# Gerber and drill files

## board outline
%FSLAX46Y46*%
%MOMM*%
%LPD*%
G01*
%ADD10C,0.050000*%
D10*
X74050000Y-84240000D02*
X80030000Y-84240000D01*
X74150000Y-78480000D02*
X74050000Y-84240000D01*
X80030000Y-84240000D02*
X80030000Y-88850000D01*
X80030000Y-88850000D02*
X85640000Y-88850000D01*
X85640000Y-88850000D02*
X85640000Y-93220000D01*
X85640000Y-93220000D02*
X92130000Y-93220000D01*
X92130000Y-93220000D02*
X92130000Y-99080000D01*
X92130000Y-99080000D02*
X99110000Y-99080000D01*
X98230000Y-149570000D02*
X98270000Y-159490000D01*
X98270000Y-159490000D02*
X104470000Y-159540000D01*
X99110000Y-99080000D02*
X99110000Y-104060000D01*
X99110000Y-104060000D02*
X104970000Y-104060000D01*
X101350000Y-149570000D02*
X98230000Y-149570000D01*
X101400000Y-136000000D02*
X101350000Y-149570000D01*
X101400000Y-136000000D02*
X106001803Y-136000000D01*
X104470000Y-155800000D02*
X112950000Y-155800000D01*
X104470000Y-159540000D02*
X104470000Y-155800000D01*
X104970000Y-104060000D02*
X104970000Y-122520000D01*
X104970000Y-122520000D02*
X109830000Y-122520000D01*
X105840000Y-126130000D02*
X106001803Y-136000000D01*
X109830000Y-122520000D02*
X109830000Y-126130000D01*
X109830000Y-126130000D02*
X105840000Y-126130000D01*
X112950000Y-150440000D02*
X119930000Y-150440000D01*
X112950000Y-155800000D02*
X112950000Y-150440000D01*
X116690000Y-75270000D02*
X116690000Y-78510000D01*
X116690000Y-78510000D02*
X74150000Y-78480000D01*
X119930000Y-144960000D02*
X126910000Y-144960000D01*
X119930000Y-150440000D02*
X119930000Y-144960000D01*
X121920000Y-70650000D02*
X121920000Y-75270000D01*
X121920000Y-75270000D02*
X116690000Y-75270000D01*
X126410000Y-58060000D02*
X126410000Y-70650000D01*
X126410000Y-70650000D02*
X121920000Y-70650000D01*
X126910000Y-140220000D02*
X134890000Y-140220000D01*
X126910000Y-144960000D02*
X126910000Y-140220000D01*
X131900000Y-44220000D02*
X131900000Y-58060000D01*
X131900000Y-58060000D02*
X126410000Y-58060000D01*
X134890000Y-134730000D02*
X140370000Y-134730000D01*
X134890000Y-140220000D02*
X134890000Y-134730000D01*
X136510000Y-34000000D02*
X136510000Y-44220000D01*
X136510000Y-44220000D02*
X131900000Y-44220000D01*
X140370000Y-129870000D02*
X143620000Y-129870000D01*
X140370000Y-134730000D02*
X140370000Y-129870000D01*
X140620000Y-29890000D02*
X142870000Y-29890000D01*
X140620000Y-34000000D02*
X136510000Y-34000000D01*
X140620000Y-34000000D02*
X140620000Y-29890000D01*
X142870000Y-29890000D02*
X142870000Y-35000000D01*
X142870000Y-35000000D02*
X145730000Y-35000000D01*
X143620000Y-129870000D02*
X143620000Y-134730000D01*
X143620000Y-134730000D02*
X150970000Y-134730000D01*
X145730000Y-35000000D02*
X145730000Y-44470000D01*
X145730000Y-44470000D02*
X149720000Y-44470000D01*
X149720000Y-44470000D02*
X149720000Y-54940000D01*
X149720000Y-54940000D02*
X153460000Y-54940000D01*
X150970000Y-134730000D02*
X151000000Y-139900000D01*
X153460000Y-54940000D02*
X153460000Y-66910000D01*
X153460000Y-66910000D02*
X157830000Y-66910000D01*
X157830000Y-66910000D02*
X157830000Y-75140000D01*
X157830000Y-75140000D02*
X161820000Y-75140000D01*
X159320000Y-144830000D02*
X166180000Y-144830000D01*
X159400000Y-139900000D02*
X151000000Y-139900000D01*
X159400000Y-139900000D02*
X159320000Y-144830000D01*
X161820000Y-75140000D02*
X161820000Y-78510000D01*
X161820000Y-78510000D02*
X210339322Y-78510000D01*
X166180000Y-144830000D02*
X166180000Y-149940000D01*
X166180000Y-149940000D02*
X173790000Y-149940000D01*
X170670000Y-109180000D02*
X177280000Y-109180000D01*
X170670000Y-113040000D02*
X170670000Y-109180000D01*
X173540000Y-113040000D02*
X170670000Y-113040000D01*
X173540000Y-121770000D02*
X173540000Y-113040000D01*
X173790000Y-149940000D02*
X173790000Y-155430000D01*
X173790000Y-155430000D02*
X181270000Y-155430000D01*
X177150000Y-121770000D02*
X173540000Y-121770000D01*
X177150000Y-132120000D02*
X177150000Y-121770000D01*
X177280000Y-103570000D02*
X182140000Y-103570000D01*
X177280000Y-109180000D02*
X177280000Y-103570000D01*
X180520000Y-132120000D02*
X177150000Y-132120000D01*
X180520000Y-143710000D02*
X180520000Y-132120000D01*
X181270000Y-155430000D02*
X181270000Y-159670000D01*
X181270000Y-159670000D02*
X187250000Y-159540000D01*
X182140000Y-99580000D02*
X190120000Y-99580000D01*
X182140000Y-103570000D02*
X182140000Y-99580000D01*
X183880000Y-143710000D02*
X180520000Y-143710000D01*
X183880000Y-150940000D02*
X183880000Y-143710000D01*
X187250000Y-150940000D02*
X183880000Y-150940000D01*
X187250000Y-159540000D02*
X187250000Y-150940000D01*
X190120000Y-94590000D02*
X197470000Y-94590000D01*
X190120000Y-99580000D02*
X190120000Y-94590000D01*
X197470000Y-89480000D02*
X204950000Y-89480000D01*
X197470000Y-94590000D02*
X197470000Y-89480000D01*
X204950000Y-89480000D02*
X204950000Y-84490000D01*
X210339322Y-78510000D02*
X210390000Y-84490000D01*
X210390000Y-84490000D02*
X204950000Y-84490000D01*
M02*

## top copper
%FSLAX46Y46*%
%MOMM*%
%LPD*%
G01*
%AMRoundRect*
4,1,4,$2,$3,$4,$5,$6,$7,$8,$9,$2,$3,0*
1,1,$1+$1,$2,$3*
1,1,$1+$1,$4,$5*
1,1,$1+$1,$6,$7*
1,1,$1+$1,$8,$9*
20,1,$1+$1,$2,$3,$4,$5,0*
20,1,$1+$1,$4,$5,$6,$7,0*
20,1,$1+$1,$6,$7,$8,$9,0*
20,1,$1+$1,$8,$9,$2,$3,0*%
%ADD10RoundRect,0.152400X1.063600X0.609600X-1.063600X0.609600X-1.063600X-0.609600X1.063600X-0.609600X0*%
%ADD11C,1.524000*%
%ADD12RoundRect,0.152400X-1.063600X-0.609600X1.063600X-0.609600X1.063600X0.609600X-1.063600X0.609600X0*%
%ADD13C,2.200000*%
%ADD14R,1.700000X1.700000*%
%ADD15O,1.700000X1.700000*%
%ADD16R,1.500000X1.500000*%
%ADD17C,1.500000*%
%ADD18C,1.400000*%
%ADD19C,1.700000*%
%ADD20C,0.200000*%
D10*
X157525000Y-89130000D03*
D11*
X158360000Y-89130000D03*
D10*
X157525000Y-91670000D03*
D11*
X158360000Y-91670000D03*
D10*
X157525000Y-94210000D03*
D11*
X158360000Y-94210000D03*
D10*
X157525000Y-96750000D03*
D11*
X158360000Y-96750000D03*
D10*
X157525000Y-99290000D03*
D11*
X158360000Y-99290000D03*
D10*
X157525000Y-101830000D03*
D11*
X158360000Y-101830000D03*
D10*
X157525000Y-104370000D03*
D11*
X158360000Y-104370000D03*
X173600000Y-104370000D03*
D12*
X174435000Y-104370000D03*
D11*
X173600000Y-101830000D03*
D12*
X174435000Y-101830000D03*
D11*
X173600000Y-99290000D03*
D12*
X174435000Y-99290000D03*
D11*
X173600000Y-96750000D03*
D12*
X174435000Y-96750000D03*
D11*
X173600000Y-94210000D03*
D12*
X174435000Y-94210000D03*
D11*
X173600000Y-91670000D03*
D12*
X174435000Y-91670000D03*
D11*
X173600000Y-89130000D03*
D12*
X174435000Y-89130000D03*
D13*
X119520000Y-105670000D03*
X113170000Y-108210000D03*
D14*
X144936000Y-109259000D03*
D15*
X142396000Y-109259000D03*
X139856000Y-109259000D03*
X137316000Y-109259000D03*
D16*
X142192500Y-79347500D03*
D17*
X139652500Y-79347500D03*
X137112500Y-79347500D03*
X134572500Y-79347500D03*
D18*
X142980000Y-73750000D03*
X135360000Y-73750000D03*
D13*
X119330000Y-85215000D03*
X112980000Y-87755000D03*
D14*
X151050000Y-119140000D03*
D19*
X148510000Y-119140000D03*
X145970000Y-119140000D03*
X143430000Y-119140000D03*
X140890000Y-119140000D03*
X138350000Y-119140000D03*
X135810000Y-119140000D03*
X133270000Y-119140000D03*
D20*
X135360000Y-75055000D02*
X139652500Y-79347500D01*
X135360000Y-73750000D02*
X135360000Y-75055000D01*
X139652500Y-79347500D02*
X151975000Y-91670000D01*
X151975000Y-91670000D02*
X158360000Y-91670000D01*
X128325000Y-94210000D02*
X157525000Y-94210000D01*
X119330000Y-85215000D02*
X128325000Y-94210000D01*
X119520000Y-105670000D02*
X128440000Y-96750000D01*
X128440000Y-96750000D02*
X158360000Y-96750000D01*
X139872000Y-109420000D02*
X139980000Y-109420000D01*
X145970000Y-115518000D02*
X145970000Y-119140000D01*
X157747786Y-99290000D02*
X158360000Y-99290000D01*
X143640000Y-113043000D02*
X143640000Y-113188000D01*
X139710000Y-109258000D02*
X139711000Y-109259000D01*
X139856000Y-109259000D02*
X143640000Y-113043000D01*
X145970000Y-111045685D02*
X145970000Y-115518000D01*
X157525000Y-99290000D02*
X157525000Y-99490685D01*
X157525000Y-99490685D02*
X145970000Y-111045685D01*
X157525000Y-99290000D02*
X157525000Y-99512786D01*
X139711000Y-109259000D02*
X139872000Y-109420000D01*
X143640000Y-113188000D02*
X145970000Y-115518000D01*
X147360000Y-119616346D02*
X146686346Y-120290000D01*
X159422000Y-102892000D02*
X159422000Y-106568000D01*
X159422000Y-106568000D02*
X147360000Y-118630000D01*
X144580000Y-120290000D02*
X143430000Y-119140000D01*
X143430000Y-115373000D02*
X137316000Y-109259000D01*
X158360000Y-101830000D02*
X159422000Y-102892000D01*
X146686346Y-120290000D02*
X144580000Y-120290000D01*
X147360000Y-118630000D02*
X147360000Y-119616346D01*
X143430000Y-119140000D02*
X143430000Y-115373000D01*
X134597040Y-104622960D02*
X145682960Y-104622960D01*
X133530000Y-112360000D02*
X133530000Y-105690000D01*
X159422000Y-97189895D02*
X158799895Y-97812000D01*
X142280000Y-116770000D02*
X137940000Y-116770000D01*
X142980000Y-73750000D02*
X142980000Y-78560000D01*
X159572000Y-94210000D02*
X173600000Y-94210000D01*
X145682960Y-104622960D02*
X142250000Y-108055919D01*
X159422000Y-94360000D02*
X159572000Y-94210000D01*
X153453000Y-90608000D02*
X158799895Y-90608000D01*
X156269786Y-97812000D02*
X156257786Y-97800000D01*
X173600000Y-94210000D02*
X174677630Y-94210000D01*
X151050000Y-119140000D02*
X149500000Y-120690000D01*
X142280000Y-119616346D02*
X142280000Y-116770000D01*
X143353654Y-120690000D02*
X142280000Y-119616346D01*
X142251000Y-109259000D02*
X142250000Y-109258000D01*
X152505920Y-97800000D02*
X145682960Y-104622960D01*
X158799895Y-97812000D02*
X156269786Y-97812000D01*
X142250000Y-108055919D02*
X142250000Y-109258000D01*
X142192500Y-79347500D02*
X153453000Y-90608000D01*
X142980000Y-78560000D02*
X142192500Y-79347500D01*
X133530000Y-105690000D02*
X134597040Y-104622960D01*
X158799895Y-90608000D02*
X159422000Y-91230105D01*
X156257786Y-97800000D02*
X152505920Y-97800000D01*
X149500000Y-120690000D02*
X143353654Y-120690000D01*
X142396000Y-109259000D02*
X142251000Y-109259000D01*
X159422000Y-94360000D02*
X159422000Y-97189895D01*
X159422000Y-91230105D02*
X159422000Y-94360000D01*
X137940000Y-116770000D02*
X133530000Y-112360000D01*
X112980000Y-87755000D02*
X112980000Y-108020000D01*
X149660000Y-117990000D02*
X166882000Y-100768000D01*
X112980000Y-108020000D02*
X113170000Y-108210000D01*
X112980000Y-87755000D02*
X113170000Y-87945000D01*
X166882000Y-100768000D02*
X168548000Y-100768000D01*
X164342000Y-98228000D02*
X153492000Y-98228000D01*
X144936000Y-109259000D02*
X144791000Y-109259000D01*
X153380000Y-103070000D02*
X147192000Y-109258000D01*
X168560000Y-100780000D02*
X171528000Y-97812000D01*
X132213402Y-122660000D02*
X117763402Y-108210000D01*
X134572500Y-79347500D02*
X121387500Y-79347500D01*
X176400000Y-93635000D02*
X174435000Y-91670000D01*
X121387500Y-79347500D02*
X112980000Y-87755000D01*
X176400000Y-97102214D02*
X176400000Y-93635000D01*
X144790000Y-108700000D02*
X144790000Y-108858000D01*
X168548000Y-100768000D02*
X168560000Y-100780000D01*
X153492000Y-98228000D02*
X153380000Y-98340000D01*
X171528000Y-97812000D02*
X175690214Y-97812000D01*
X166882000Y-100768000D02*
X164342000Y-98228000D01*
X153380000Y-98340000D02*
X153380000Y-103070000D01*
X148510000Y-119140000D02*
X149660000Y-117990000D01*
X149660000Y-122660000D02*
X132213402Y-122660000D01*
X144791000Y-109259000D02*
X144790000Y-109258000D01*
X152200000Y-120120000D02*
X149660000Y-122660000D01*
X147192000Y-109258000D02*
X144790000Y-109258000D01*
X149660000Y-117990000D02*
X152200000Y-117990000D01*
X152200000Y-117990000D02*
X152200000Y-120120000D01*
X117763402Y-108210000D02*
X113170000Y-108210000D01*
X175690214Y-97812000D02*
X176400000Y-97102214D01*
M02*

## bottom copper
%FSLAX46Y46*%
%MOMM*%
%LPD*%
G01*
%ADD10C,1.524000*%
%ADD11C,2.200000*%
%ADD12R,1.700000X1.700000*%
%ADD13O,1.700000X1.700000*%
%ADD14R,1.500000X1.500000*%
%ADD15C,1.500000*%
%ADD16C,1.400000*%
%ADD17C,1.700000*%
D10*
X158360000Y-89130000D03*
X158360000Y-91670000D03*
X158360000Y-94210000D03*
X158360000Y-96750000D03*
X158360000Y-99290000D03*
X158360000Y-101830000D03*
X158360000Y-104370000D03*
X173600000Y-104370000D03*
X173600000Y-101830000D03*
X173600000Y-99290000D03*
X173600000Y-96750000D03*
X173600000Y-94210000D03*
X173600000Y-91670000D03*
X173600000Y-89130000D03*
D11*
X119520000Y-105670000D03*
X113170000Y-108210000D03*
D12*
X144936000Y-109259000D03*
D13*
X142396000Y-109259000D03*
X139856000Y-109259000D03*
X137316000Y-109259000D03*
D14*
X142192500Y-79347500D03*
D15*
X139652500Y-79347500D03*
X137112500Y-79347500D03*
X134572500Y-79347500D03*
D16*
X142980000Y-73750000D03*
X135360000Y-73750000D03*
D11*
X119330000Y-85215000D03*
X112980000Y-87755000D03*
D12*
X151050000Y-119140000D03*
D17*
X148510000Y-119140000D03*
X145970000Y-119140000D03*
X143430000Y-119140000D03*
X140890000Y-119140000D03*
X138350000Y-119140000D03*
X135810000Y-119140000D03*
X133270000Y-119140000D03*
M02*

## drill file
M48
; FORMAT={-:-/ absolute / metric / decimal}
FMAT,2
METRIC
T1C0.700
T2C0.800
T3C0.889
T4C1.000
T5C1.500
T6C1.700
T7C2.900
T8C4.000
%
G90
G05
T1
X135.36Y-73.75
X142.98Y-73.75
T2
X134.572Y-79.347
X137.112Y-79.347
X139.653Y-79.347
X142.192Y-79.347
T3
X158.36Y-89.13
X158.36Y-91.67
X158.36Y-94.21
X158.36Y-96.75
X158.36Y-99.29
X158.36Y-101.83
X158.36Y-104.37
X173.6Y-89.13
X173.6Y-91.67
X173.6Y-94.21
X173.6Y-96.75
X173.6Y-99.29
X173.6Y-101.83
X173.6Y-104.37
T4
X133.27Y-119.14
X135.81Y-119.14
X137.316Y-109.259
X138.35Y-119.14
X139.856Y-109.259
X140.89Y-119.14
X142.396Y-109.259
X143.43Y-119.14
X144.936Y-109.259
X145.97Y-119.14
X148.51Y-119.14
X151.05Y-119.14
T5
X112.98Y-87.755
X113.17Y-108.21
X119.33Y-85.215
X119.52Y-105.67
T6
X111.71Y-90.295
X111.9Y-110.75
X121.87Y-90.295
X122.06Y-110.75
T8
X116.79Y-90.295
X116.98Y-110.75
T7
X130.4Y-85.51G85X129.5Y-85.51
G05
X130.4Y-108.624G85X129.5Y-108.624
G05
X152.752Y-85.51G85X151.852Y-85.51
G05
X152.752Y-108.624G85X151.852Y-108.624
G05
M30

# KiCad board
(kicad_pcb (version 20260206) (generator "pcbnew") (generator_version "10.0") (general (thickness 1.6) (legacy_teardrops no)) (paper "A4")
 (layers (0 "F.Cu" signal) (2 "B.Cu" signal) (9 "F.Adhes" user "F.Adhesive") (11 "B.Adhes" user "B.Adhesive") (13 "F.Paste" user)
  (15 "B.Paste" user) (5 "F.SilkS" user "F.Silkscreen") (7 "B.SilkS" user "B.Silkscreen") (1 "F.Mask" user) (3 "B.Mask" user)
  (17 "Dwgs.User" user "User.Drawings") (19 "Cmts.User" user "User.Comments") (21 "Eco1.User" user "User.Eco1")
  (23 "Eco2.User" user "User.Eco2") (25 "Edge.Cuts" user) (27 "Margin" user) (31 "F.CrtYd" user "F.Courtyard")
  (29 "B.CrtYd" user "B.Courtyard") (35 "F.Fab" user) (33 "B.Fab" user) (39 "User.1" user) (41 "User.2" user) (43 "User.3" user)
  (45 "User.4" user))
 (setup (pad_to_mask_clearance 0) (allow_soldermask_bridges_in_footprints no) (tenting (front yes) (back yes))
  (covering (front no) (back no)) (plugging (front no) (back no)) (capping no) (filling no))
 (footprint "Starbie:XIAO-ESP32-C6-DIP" (layer "F.Cu") (at 165.98 96.75 90)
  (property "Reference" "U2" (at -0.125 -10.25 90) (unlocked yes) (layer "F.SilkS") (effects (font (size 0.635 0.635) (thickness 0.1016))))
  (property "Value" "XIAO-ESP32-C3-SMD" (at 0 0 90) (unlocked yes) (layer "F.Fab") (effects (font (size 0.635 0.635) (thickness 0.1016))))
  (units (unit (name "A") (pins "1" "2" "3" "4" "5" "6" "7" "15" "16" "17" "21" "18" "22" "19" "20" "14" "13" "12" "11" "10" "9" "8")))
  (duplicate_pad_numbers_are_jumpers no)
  (pad "1" smd roundrect (at 7.62 -8.455 180) (size 2.432 1.524) (layers "F.Cu" "F.Mask") (roundrect_rratio 0.1)
   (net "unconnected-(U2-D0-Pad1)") (thermal_bridge_angle 45))
  (pad "1" thru_hole circle (at 7.62 -7.62 180) (size 1.524 1.524) (drill 0.889) (layers "*.Cu" "*.Mask") (remove_unused_layers no)
   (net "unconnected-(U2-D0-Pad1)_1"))
  (pad "2" smd roundrect (at 5.08 -8.455 180) (size 2.432 1.524) (layers "F.Cu" "F.Mask") (roundrect_rratio 0.1) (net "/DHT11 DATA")
   (thermal_bridge_angle 45))
  (pad "2" thru_hole circle (at 5.08 -7.62 180) (size 1.524 1.524) (drill 0.889) (layers "*.Cu" "*.Mask") (remove_unused_layers no)
   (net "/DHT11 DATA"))
  (pad "3" smd roundrect (at 2.54 -8.455 180) (size 2.432 1.524) (layers "F.Cu" "F.Mask") (roundrect_rratio 0.1) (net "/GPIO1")
   (thermal_bridge_angle 45))
  (pad "3" thru_hole circle (at 2.54 -7.62 180) (size 1.524 1.524) (drill 0.889) (layers "*.Cu" "*.Mask") (remove_unused_layers no)
   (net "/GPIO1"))
  (pad "4" smd roundrect (at 0 -8.455 180) (size 2.432 1.524) (layers "F.Cu" "F.Mask") (roundrect_rratio 0.1) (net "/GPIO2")
   (thermal_bridge_angle 45))
  (pad "4" thru_hole circle (at 0 -7.62 180) (size 1.524 1.524) (drill 0.889) (layers "*.Cu" "*.Mask") (remove_unused_layers no)
   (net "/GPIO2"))
  (pad "5" smd roundrect (at -2.54 -8.455 180) (size 2.432 1.524) (layers "F.Cu" "F.Mask") (roundrect_rratio 0.1) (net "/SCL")
   (thermal_bridge_angle 45))
  (pad "5" thru_hole circle (at -2.54 -7.62 180) (size 1.524 1.524) (drill 0.889) (layers "*.Cu" "*.Mask") (remove_unused_layers no)
   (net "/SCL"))
  (pad "6" smd roundrect (at -5.08 -8.455 180) (size 2.432 1.524) (layers "F.Cu" "F.Mask") (roundrect_rratio 0.1) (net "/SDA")
   (thermal_bridge_angle 45))
  (pad "6" thru_hole circle (at -5.08 -7.62 180) (size 1.524 1.524) (drill 0.889) (layers "*.Cu" "*.Mask") (remove_unused_layers no)
   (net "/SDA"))
  (pad "7" smd roundrect (at -7.62 -8.455 180) (size 2.432 1.524) (layers "F.Cu" "F.Mask") (roundrect_rratio 0.1)
   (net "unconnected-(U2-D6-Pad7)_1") (thermal_bridge_angle 45))
  (pad "7" thru_hole circle (at -7.62 -7.62 180) (size 1.524 1.524) (drill 0.889) (layers "*.Cu" "*.Mask") (remove_unused_layers no)
   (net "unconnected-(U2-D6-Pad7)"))
  (pad "8" thru_hole circle (at -7.62 7.62) (size 1.524 1.524) (drill 0.889) (layers "*.Cu" "*.Mask") (remove_unused_layers no)
   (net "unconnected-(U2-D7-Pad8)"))
  (pad "8" smd roundrect (at -7.62 8.455) (size 2.432 1.524) (layers "F.Cu" "F.Mask") (roundrect_rratio 0.1)
   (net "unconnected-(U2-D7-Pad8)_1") (thermal_bridge_angle 45))
  (pad "9" thru_hole circle (at -5.08 7.62) (size 1.524 1.524) (drill 0.889) (layers "*.Cu" "*.Mask") (remove_unused_layers no)
   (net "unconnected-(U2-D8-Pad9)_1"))
  (pad "9" smd roundrect (at -5.08 8.455) (size 2.432 1.524) (layers "F.Cu" "F.Mask") (roundrect_rratio 0.1)
   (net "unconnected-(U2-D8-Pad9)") (thermal_bridge_angle 45))
  (pad "10" thru_hole circle (at -2.54 7.62) (size 1.524 1.524) (drill 0.889) (layers "*.Cu" "*.Mask") (remove_unused_layers no)
   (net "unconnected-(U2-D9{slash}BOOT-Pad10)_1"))
  (pad "10" smd roundrect (at -2.54 8.455) (size 2.432 1.524) (layers "F.Cu" "F.Mask") (roundrect_rratio 0.1)
   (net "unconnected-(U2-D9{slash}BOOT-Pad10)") (thermal_bridge_angle 45))
  (pad "11" thru_hole circle (at 0 7.62) (size 1.524 1.524) (drill 0.889) (layers "*.Cu" "*.Mask") (remove_unused_layers no)
   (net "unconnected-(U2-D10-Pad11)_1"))
  (pad "11" smd roundrect (at 0 8.455) (size 2.432 1.524) (layers "F.Cu" "F.Mask") (roundrect_rratio 0.1) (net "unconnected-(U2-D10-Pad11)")
   (thermal_bridge_angle 45))
  (pad "12" thru_hole circle (at 2.54 7.62) (size 1.524 1.524) (drill 0.889) (layers "*.Cu" "*.Mask") (remove_unused_layers no)
   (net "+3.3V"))
  (pad "12" smd roundrect (at 2.54 8.455) (size 2.432 1.524) (layers "F.Cu" "F.Mask") (roundrect_rratio 0.1) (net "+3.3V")
   (thermal_bridge_angle 45))
  (pad "13" thru_hole circle (at 5.08 7.62) (size 1.524 1.524) (drill 0.889) (layers "*.Cu" "*.Mask") (remove_unused_layers no) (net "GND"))
  (pad "13" smd roundrect (at 5.08 8.455) (size 2.432 1.524) (layers "F.Cu" "F.Mask") (roundrect_rratio 0.1) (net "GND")
   (thermal_bridge_angle 45))
  (pad "14" thru_hole circle (at 7.62 7.62) (size 1.524 1.524) (drill 0.889) (layers "*.Cu" "*.Mask") (remove_unused_layers no) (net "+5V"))
  (pad "14" smd roundrect (at 7.62 8.455) (size 2.432 1.524) (layers "F.Cu" "F.Mask") (roundrect_rratio 0.1) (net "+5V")
   (thermal_bridge_angle 45)))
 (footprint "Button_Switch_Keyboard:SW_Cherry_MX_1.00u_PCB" (layer "F.Cu") (at 119.52 105.67)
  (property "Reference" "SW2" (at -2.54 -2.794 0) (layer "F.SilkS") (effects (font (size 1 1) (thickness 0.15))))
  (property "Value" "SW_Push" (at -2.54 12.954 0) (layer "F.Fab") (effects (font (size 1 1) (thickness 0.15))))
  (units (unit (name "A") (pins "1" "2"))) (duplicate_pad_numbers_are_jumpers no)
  (pad "" np_thru_hole circle (at -7.62 5.08) (size 1.7 1.7) (drill 1.7) (layers "*.Cu" "*.Mask"))
  (pad "" np_thru_hole circle (at -2.54 5.08) (size 4 4) (drill 4) (layers "*.Cu" "*.Mask"))
  (pad "" np_thru_hole circle (at 2.54 5.08) (size 1.7 1.7) (drill 1.7) (layers "*.Cu" "*.Mask"))
  (pad "1" thru_hole circle (at 0 0) (size 2.2 2.2) (drill 1.5) (layers "*.Cu" "*.Mask") (remove_unused_layers no) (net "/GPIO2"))
  (pad "2" thru_hole circle (at -6.35 2.54) (size 2.2 2.2) (drill 1.5) (layers "*.Cu" "*.Mask") (remove_unused_layers no) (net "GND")))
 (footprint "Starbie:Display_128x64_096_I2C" (layer "F.Cu") (at 141.126 109.259 180)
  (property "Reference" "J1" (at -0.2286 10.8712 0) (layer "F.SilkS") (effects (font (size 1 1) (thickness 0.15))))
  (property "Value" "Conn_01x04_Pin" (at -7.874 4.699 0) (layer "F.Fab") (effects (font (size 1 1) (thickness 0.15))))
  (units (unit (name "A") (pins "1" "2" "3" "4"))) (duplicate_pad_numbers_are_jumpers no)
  (pad "" np_thru_hole oval (at -11.176 0.635 180) (size 3.8 2.9) (drill oval 3.8 2.9) (layers "*.Cu" "*.Mask"))
  (pad "" np_thru_hole oval (at -11.176 23.749 180) (size 3.8 2.9) (drill oval 3.8 2.9) (layers "*.Cu" "*.Mask"))
  (pad "" np_thru_hole oval (at 11.176 0.635 180) (size 3.8 2.9) (drill oval 3.8 2.9) (layers "*.Cu" "*.Mask"))
  (pad "" np_thru_hole oval (at 11.176 23.749 180) (size 3.8 2.9) (drill oval 3.8 2.9) (layers "*.Cu" "*.Mask"))
  (pad "1" thru_hole rect (at -3.81 0 270) (size 1.7 1.7) (drill 1) (layers "*.Cu" "*.Mask") (remove_unused_layers no) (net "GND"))
  (pad "2" thru_hole oval (at -1.27 0 270) (size 1.7 1.7) (drill 1) (layers "*.Cu" "*.Mask") (remove_unused_layers no) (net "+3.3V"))
  (pad "3" thru_hole oval (at 1.27 0 270) (size 1.7 1.7) (drill 1) (layers "*.Cu" "*.Mask") (remove_unused_layers no) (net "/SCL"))
  (pad "4" thru_hole oval (at 3.81 0 270) (size 1.7 1.7) (drill 1) (layers "*.Cu" "*.Mask") (remove_unused_layers no) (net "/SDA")))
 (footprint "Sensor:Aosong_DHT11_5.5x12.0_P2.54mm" (layer "F.Cu") (at 142.1925 79.3475 -90)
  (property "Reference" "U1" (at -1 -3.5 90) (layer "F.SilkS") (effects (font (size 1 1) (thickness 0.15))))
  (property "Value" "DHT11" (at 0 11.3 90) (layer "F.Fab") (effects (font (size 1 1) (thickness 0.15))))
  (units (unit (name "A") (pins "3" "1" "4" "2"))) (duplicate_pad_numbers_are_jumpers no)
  (pad "1" thru_hole rect (at 0 0 270) (size 1.5 1.5) (drill 0.8) (layers "*.Cu" "*.Mask") (remove_unused_layers no) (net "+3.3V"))
  (pad "2" thru_hole circle (at 0 2.54 270) (size 1.5 1.5) (drill 0.8) (layers "*.Cu" "*.Mask") (remove_unused_layers no)
   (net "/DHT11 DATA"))
  (pad "3" thru_hole circle (at 0 5.08 270) (size 1.5 1.5) (drill 0.8) (layers "*.Cu" "*.Mask") (remove_unused_layers no)
   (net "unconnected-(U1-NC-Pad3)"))
  (pad "4" thru_hole circle (at 0 7.62 270) (size 1.5 1.5) (drill 0.8) (layers "*.Cu" "*.Mask") (remove_unused_layers no) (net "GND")))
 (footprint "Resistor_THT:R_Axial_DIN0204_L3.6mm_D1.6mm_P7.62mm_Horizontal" (layer "F.Cu") (at 142.98 73.75 180)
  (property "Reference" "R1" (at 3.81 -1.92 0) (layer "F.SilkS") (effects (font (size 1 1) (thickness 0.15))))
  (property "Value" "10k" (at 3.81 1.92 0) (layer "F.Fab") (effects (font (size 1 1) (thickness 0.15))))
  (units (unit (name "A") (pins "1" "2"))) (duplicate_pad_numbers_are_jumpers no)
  (pad "1" thru_hole circle (at 0 0 180) (size 1.4 1.4) (drill 0.7) (layers "*.Cu" "*.Mask") (remove_unused_layers no) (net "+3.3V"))
  (pad "2" thru_hole circle (at 7.62 0 180) (size 1.4 1.4) (drill 0.7) (layers "*.Cu" "*.Mask") (remove_unused_layers no)
   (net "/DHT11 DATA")))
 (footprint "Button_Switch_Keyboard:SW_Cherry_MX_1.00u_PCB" (layer "F.Cu") (at 119.33 85.215)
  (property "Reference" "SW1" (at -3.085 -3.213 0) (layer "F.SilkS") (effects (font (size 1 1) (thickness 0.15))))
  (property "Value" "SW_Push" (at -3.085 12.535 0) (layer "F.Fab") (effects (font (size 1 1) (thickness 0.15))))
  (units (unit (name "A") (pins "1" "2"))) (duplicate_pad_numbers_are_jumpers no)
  (pad "" np_thru_hole circle (at -7.62 5.08) (size 1.7 1.7) (drill 1.7) (layers "*.Cu" "*.Mask"))
  (pad "" np_thru_hole circle (at -2.54 5.08) (size 4 4) (drill 4) (layers "*.Cu" "*.Mask"))
  (pad "" np_thru_hole circle (at 2.54 5.08) (size 1.7 1.7) (drill 1.7) (layers "*.Cu" "*.Mask"))
  (pad "1" thru_hole circle (at 0 0) (size 2.2 2.2) (drill 1.5) (layers "*.Cu" "*.Mask") (remove_unused_layers no) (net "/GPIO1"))
  (pad "2" thru_hole circle (at -6.35 2.54) (size 2.2 2.2) (drill 1.5) (layers "*.Cu" "*.Mask") (remove_unused_layers no) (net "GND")))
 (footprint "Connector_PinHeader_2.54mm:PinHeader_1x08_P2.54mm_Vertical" (layer "F.Cu") (at 151.05 119.14 -90)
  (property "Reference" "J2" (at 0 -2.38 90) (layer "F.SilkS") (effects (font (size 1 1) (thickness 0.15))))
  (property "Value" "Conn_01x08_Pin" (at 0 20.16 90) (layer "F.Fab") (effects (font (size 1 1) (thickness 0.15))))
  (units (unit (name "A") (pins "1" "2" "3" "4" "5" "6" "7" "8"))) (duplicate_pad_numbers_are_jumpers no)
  (pad "1" thru_hole rect (at 0 0 270) (size 1.7 1.7) (drill 1) (layers "*.Cu" "*.Mask") (remove_unused_layers no) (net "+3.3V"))
  (pad "2" thru_hole circle (at 0 2.54 270) (size 1.7 1.7) (drill 1) (layers "*.Cu" "*.Mask") (remove_unused_layers no) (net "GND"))
  (pad "3" thru_hole circle (at 0 5.08 270) (size 1.7 1.7) (drill 1) (layers "*.Cu" "*.Mask") (remove_unused_layers no) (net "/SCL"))
  (pad "4" thru_hole circle (at 0 7.62 270) (size 1.7 1.7) (drill 1) (layers "*.Cu" "*.Mask") (remove_unused_layers no) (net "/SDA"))
  (pad "5" thru_hole circle (at 0 10.16 270) (size 1.7 1.7) (drill 1) (layers "*.Cu" "*.Mask") (remove_unused_layers no)
   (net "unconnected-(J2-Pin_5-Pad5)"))
  (pad "6" thru_hole circle (at 0 12.7 270) (size 1.7 1.7) (drill 1) (layers "*.Cu" "*.Mask") (remove_unused_layers no)
   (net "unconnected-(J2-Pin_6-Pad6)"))
  (pad "7" thru_hole circle (at 0 15.24 270) (size 1.7 1.7) (drill 1) (layers "*.Cu" "*.Mask") (remove_unused_layers no)
   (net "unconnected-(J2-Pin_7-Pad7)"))
  (pad "8" thru_hole circle (at 0 17.78 270) (size 1.7 1.7) (drill 1) (layers "*.Cu" "*.Mask") (remove_unused_layers no)
   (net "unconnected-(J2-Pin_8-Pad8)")))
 (gr_line (start 74.05 84.24) (end 80.03 84.24) (stroke (width 0.05) (type default)) (layer "Edge.Cuts"))
 (gr_line (start 74.15 78.48) (end 74.05 84.24) (stroke (width 0.05) (type default)) (layer "Edge.Cuts"))
 (gr_line (start 80.03 84.24) (end 80.03 88.85) (stroke (width 0.05) (type default)) (layer "Edge.Cuts"))
 (gr_line (start 80.03 88.85) (end 85.64 88.85) (stroke (width 0.05) (type default)) (layer "Edge.Cuts"))
 (gr_line (start 85.64 88.85) (end 85.64 93.22) (stroke (width 0.05) (type default)) (layer "Edge.Cuts"))
 (gr_line (start 85.64 93.22) (end 92.13 93.22) (stroke (width 0.05) (type default)) (layer "Edge.Cuts"))
 (gr_line (start 92.13 93.22) (end 92.13 99.08) (stroke (width 0.05) (type default)) (layer "Edge.Cuts"))
 (gr_line (start 92.13 99.08) (end 99.11 99.08) (stroke (width 0.05) (type default)) (layer "Edge.Cuts"))
 (gr_line (start 98.23 149.57) (end 98.27 159.49) (stroke (width 0.05) (type default)) (layer "Edge.Cuts"))
 (gr_line (start 98.27 159.49) (end 104.47 159.54) (stroke (width 0.05) (type default)) (layer "Edge.Cuts"))
 (gr_line (start 99.11 99.08) (end 99.11 104.06) (stroke (width 0.05) (type default)) (layer "Edge.Cuts"))
 (gr_line (start 99.11 104.06) (end 104.97 104.06) (stroke (width 0.05) (type default)) (layer "Edge.Cuts"))
 (gr_line (start 101.35 149.57) (end 98.23 149.57) (stroke (width 0.05) (type default)) (layer "Edge.Cuts"))
 (gr_line (start 101.4 136) (end 101.35 149.57) (stroke (width 0.05) (type default)) (layer "Edge.Cuts"))
 (gr_line (start 101.4 136) (end 106.001803 136) (stroke (width 0.05) (type default)) (layer "Edge.Cuts"))
 (gr_line (start 104.47 155.8) (end 112.95 155.8) (stroke (width 0.05) (type default)) (layer "Edge.Cuts"))
 (gr_line (start 104.47 159.54) (end 104.47 155.8) (stroke (width 0.05) (type default)) (layer "Edge.Cuts"))
 (gr_line (start 104.97 104.06) (end 104.97 122.52) (stroke (width 0.05) (type default)) (layer "Edge.Cuts"))
 (gr_line (start 104.97 122.52) (end 109.83 122.52) (stroke (width 0.05) (type default)) (layer "Edge.Cuts"))
 (gr_line (start 105.84 126.13) (end 106.001803 136) (stroke (width 0.05) (type default)) (layer "Edge.Cuts"))
 (gr_line (start 109.83 122.52) (end 109.83 126.13) (stroke (width 0.05) (type default)) (layer "Edge.Cuts"))
 (gr_line (start 109.83 126.13) (end 105.84 126.13) (stroke (width 0.05) (type default)) (layer "Edge.Cuts"))
 (gr_line (start 112.95 150.44) (end 119.93 150.44) (stroke (width 0.05) (type default)) (layer "Edge.Cuts"))
 (gr_line (start 112.95 155.8) (end 112.95 150.44) (stroke (width 0.05) (type default)) (layer "Edge.Cuts"))
 (gr_line (start 116.69 75.27) (end 116.69 78.51) (stroke (width 0.05) (type default)) (layer "Edge.Cuts"))
 (gr_line (start 116.69 78.51) (end 74.15 78.48) (stroke (width 0.05) (type default)) (layer "Edge.Cuts"))
 (gr_line (start 119.93 144.96) (end 126.91 144.96) (stroke (width 0.05) (type default)) (layer "Edge.Cuts"))
 (gr_line (start 119.93 150.44) (end 119.93 144.96) (stroke (width 0.05) (type default)) (layer "Edge.Cuts"))
 (gr_line (start 121.92 70.65) (end 121.92 75.27) (stroke (width 0.05) (type default)) (layer "Edge.Cuts"))
 (gr_line (start 121.92 75.27) (end 116.69 75.27) (stroke (width 0.05) (type default)) (layer "Edge.Cuts"))
 (gr_line (start 126.41 58.06) (end 126.41 70.65) (stroke (width 0.05) (type default)) (layer "Edge.Cuts"))
 (gr_line (start 126.41 70.65) (end 121.92 70.65) (stroke (width 0.05) (type default)) (layer "Edge.Cuts"))
 (gr_line (start 126.91 140.22) (end 134.89 140.22) (stroke (width 0.05) (type default)) (layer "Edge.Cuts"))
 (gr_line (start 126.91 144.96) (end 126.91 140.22) (stroke (width 0.05) (type default)) (layer "Edge.Cuts"))
 (gr_line (start 131.9 44.22) (end 131.9 58.06) (stroke (width 0.05) (type default)) (layer "Edge.Cuts"))
 (gr_line (start 131.9 58.06) (end 126.41 58.06) (stroke (width 0.05) (type default)) (layer "Edge.Cuts"))
 (gr_line (start 134.89 134.73) (end 140.37 134.73) (stroke (width 0.05) (type default)) (layer "Edge.Cuts"))
 (gr_line (start 134.89 140.22) (end 134.89 134.73) (stroke (width 0.05) (type default)) (layer "Edge.Cuts"))
 (gr_line (start 136.51 34) (end 136.51 44.22) (stroke (width 0.05) (type default)) (layer "Edge.Cuts"))
 (gr_line (start 136.51 44.22) (end 131.9 44.22) (stroke (width 0.05) (type default)) (layer "Edge.Cuts"))
 (gr_line (start 140.37 129.87) (end 143.62 129.87) (stroke (width 0.05) (type default)) (layer "Edge.Cuts"))
 (gr_line (start 140.37 134.73) (end 140.37 129.87) (stroke (width 0.05) (type default)) (layer "Edge.Cuts"))
 (gr_line (start 140.62 29.89) (end 142.87 29.89) (stroke (width 0.05) (type default)) (layer "Edge.Cuts"))
 (gr_line (start 140.62 34) (end 136.51 34) (stroke (width 0.05) (type default)) (layer "Edge.Cuts"))
 (gr_line (start 140.62 34) (end 140.62 29.89) (stroke (width 0.05) (type default)) (layer "Edge.Cuts"))
 (gr_line (start 142.87 29.89) (end 142.87 35) (stroke (width 0.05) (type default)) (layer "Edge.Cuts"))
 (gr_line (start 142.87 35) (end 145.73 35) (stroke (width 0.05) (type default)) (layer "Edge.Cuts"))
 (gr_line (start 143.62 129.87) (end 143.62 134.73) (stroke (width 0.05) (type default)) (layer "Edge.Cuts"))
 (gr_line (start 143.62 134.73) (end 150.97 134.73) (stroke (width 0.05) (type default)) (layer "Edge.Cuts"))
 (gr_line (start 145.73 35) (end 145.73 44.47) (stroke (width 0.05) (type default)) (layer "Edge.Cuts"))
 (gr_line (start 145.73 44.47) (end 149.72 44.47) (stroke (width 0.05) (type default)) (layer "Edge.Cuts"))
 (gr_line (start 149.72 44.47) (end 149.72 54.94) (stroke (width 0.05) (type default)) (layer "Edge.Cuts"))
 (gr_line (start 149.72 54.94) (end 153.46 54.94) (stroke (width 0.05) (type default)) (layer "Edge.Cuts"))
 (gr_line (start 150.97 134.73) (end 151 139.9) (stroke (width 0.05) (type default)) (layer "Edge.Cuts"))
 (gr_line (start 153.46 54.94) (end 153.46 66.91) (stroke (width 0.05) (type default)) (layer "Edge.Cuts"))
 (gr_line (start 153.46 66.91) (end 157.83 66.91) (stroke (width 0.05) (type default)) (layer "Edge.Cuts"))
 (gr_line (start 157.83 66.91) (end 157.83 75.14) (stroke (width 0.05) (type default)) (layer "Edge.Cuts"))
 (gr_line (start 157.83 75.14) (end 161.82 75.14) (stroke (width 0.05) (type default)) (layer "Edge.Cuts"))
 (gr_line (start 159.32 144.83) (end 166.18 144.83) (stroke (width 0.05) (type default)) (layer "Edge.Cuts"))
 (gr_line (start 159.4 139.9) (end 151 139.9) (stroke (width 0.05) (type default)) (layer "Edge.Cuts"))
 (gr_line (start 159.4 139.9) (end 159.32 144.83) (stroke (width 0.05) (type default)) (layer "Edge.Cuts"))
 (gr_line (start 161.82 75.14) (end 161.82 78.51) (stroke (width 0.05) (type default)) (layer "Edge.Cuts"))
 (gr_line (start 161.82 78.51) (end 210.339322 78.51) (stroke (width 0.05) (type default)) (layer "Edge.Cuts"))
 (gr_line (start 166.18 144.83) (end 166.18 149.94) (stroke (width 0.05) (type default)) (layer "Edge.Cuts"))
 (gr_line (start 166.18 149.94) (end 173.79 149.94) (stroke (width 0.05) (type default)) (layer "Edge.Cuts"))
 (gr_line (start 170.67 109.18) (end 177.28 109.18) (stroke (width 0.05) (type default)) (layer "Edge.Cuts"))
 (gr_line (start 170.67 113.04) (end 170.67 109.18) (stroke (width 0.05) (type default)) (layer "Edge.Cuts"))
 (gr_line (start 173.54 113.04) (end 170.67 113.04) (stroke (width 0.05) (type default)) (layer "Edge.Cuts"))
 (gr_line (start 173.54 121.77) (end 173.54 113.04) (stroke (width 0.05) (type default)) (layer "Edge.Cuts"))
 (gr_line (start 173.79 149.94) (end 173.79 155.43) (stroke (width 0.05) (type default)) (layer "Edge.Cuts"))
 (gr_line (start 173.79 155.43) (end 181.27 155.43) (stroke (width 0.05) (type default)) (layer "Edge.Cuts"))
 (gr_line (start 177.15 121.77) (end 173.54 121.77) (stroke (width 0.05) (type default)) (layer "Edge.Cuts"))
 (gr_line (start 177.15 132.12) (end 177.15 121.77) (stroke (width 0.05) (type default)) (layer "Edge.Cuts"))
 (gr_line (start 177.28 103.57) (end 182.14 103.57) (stroke (width 0.05) (type default)) (layer "Edge.Cuts"))
 (gr_line (start 177.28 109.18) (end 177.28 103.57) (stroke (width 0.05) (type default)) (layer "Edge.Cuts"))
 (gr_line (start 180.52 132.12) (end 177.15 132.12) (stroke (width 0.05) (type default)) (layer "Edge.Cuts"))
 (gr_line (start 180.52 143.71) (end 180.52 132.12) (stroke (width 0.05) (type default)) (layer "Edge.Cuts"))
 (gr_line (start 181.27 155.43) (end 181.27 159.67) (stroke (width 0.05) (type default)) (layer "Edge.Cuts"))
 (gr_line (start 181.27 159.67) (end 187.25 159.54) (stroke (width 0.05) (type default)) (layer "Edge.Cuts"))
 (gr_line (start 182.14 99.58) (end 190.12 99.58) (stroke (width 0.05) (type default)) (layer "Edge.Cuts"))
 (gr_line (start 182.14 103.57) (end 182.14 99.58) (stroke (width 0.05) (type default)) (layer "Edge.Cuts"))
 (gr_line (start 183.88 143.71) (end 180.52 143.71) (stroke (width 0.05) (type default)) (layer "Edge.Cuts"))
 (gr_line (start 183.88 150.94) (end 183.88 143.71) (stroke (width 0.05) (type default)) (layer "Edge.Cuts"))
 (gr_line (start 187.25 150.94) (end 183.88 150.94) (stroke (width 0.05) (type default)) (layer "Edge.Cuts"))
 (gr_line (start 187.25 159.54) (end 187.25 150.94) (stroke (width 0.05) (type default)) (layer "Edge.Cuts"))
 (gr_line (start 190.12 94.59) (end 197.47 94.59) (stroke (width 0.05) (type default)) (layer "Edge.Cuts"))
 (gr_line (start 190.12 99.58) (end 190.12 94.59) (stroke (width 0.05) (type default)) (layer "Edge.Cuts"))
 (gr_line (start 197.47 89.48) (end 204.95 89.48) (stroke (width 0.05) (type default)) (layer "Edge.Cuts"))
 (gr_line (start 197.47 94.59) (end 197.47 89.48) (stroke (width 0.05) (type default)) (layer "Edge.Cuts"))
 (gr_line (start 204.95 89.48) (end 204.95 84.49) (stroke (width 0.05) (type default)) (layer "Edge.Cuts"))
 (gr_line (start 210.339322 78.51) (end 210.39 84.49) (stroke (width 0.05) (type default)) (layer "Edge.Cuts"))
 (gr_line (start 210.39 84.49) (end 204.95 84.49) (stroke (width 0.05) (type default)) (layer "Edge.Cuts"))
 (segment (start 135.36 75.055) (end 139.6525 79.3475) (width 0.2) (layer "F.Cu") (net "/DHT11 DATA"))
 (segment (start 135.36 73.75) (end 135.36 75.055) (width 0.2) (layer "F.Cu") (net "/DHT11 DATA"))
 (segment (start 139.6525 79.3475) (end 151.975 91.67) (width 0.2) (layer "F.Cu") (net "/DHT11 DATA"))
 (segment (start 151.975 91.67) (end 158.36 91.67) (width 0.2) (layer "F.Cu") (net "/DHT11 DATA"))
 (segment (start 128.325 94.21) (end 157.525 94.21) (width 0.2) (layer "F.Cu") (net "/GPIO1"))
 (segment (start 119.33 85.215) (end 128.325 94.21) (width 0.2) (layer "F.Cu") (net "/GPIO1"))
 (segment (start 119.52 105.67) (end 128.44 96.75) (width 0.2) (layer "F.Cu") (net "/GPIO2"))
 (segment (start 128.44 96.75) (end 158.36 96.75) (width 0.2) (layer "F.Cu") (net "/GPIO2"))
 (segment (start 139.872 109.42) (end 139.98 109.42) (width 0.2) (layer "F.Cu") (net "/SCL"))
 (segment (start 145.97 115.518) (end 145.97 119.14) (width 0.2) (layer "F.Cu") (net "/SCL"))
 (segment (start 157.747786 99.29) (end 158.36 99.29) (width 0.2) (layer "F.Cu") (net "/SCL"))
 (segment (start 143.64 113.043) (end 143.64 113.188) (width 0.2) (layer "F.Cu") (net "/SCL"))
 (segment (start 139.71 109.258) (end 139.711 109.259) (width 0.2) (layer "F.Cu") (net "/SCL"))
 (segment (start 139.856 109.259) (end 143.64 113.043) (width 0.2) (layer "F.Cu") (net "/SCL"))
 (segment (start 145.97 111.045685) (end 145.97 115.518) (width 0.2) (layer "F.Cu") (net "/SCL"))
 (segment (start 157.525 99.29) (end 157.525 99.490685) (width 0.2) (layer "F.Cu") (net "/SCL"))
 (segment (start 157.525 99.490685) (end 145.97 111.045685) (width 0.2) (layer "F.Cu") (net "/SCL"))
 (segment (start 157.525 99.29) (end 157.525 99.512786) (width 0.2) (layer "F.Cu") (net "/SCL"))
 (segment (start 139.711 109.259) (end 139.872 109.42) (width 0.2) (layer "F.Cu") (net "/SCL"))
 (segment (start 143.64 113.188) (end 145.97 115.518) (width 0.2) (layer "F.Cu") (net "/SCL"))
 (segment (start 147.36 119.616346) (end 146.686346 120.29) (width 0.2) (layer "F.Cu") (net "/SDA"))
 (segment (start 159.422 102.892) (end 159.422 106.568) (width 0.2) (layer "F.Cu") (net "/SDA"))
 (segment (start 159.422 106.568) (end 147.36 118.63) (width 0.2) (layer "F.Cu") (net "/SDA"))
 (segment (start 144.58 120.29) (end 143.43 119.14) (width 0.2) (layer "F.Cu") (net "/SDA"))
 (segment (start 143.43 115.373) (end 137.316 109.259) (width 0.2) (layer "F.Cu") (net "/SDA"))
 (segment (start 158.36 101.83) (end 159.422 102.892) (width 0.2) (layer "F.Cu") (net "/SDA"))
 (segment (start 146.686346 120.29) (end 144.58 120.29) (width 0.2) (layer "F.Cu") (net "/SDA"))
 (segment (start 147.36 118.63) (end 147.36 119.616346) (width 0.2) (layer "F.Cu") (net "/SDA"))
 (segment (start 143.43 119.14) (end 143.43 115.373) (width 0.2) (layer "F.Cu") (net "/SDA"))
 (segment (start 134.59704 104.62296) (end 145.68296 104.62296) (width 0.2) (layer "F.Cu") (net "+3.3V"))
 (segment (start 133.53 112.36) (end 133.53 105.69) (width 0.2) (layer "F.Cu") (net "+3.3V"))
 (segment (start 159.422 97.189895) (end 158.799895 97.812) (width 0.2) (layer "F.Cu") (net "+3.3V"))
 (segment (start 142.28 116.77) (end 137.94 116.77) (width 0.2) (layer "F.Cu") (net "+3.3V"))
 (segment (start 142.98 73.75) (end 142.98 78.56) (width 0.2) (layer "F.Cu") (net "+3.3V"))
 (segment (start 159.572 94.21) (end 173.6 94.21) (width 0.2) (layer "F.Cu") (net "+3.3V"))
 (segment (start 145.68296 104.62296) (end 142.25 108.055919) (width 0.2) (layer "F.Cu") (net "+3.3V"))
 (segment (start 159.422 94.36) (end 159.572 94.21) (width 0.2) (layer "F.Cu") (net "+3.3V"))
 (segment (start 153.453 90.608) (end 158.799895 90.608) (width 0.2) (layer "F.Cu") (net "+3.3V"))
 (segment (start 156.269786 97.812) (end 156.257786 97.8) (width 0.2) (layer "F.Cu") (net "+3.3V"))
 (segment (start 173.6 94.21) (end 174.67763 94.21) (width 0.2) (layer "F.Cu") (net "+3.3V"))
 (segment (start 151.05 119.14) (end 149.5 120.69) (width 0.2) (layer "F.Cu") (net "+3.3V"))
 (segment (start 142.28 119.616346) (end 142.28 116.77) (width 0.2) (layer "F.Cu") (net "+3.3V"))
 (segment (start 143.353654 120.69) (end 142.28 119.616346) (width 0.2) (layer "F.Cu") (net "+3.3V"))
 (segment (start 142.251 109.259) (end 142.25 109.258) (width 0.2) (layer "F.Cu") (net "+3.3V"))
 (segment (start 152.50592 97.8) (end 145.68296 104.62296) (width 0.2) (layer "F.Cu") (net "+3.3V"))
 (segment (start 158.799895 97.812) (end 156.269786 97.812) (width 0.2) (layer "F.Cu") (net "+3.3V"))
 (segment (start 142.25 108.055919) (end 142.25 109.258) (width 0.2) (layer "F.Cu") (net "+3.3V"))
 (segment (start 142.1925 79.3475) (end 153.453 90.608) (width 0.2) (layer "F.Cu") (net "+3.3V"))
 (segment (start 142.98 78.56) (end 142.1925 79.3475) (width 0.2) (layer "F.Cu") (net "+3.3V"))
 (segment (start 133.53 105.69) (end 134.59704 104.62296) (width 0.2) (layer "F.Cu") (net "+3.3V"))
 (segment (start 158.799895 90.608) (end 159.422 91.230105) (width 0.2) (layer "F.Cu") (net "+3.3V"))
 (segment (start 156.257786 97.8) (end 152.50592 97.8) (width 0.2) (layer "F.Cu") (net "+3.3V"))
 (segment (start 149.5 120.69) (end 143.353654 120.69) (width 0.2) (layer "F.Cu") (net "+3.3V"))
 (segment (start 142.396 109.259) (end 142.251 109.259) (width 0.2) (layer "F.Cu") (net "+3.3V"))
 (segment (start 159.422 94.36) (end 159.422 97.189895) (width 0.2) (layer "F.Cu") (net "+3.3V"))
 (segment (start 159.422 91.230105) (end 159.422 94.36) (width 0.2) (layer "F.Cu") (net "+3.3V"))
 (segment (start 137.94 116.77) (end 133.53 112.36) (width 0.2) (layer "F.Cu") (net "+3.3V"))
 (segment (start 112.98 87.755) (end 112.98 108.02) (width 0.2) (layer "F.Cu") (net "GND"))
 (segment (start 149.66 117.99) (end 166.882 100.768) (width 0.2) (layer "F.Cu") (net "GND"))
 (segment (start 112.98 108.02) (end 113.17 108.21) (width 0.2) (layer "F.Cu") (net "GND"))
 (segment (start 112.98 87.755) (end 113.17 87.945) (width 0.2) (layer "F.Cu") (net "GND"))
 (segment (start 166.882 100.768) (end 168.548 100.768) (width 0.2) (layer "F.Cu") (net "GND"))
 (segment (start 164.342 98.228) (end 153.492 98.228) (width 0.2) (layer "F.Cu") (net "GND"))
 (segment (start 144.936 109.259) (end 144.791 109.259) (width 0.2) (layer "F.Cu") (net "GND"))
 (segment (start 153.38 103.07) (end 147.192 109.258) (width 0.2) (layer "F.Cu") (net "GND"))
 (segment (start 168.56 100.78) (end 171.528 97.812) (width 0.2) (layer "F.Cu") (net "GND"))
 (segment (start 132.213402 122.66) (end 117.763402 108.21) (width 0.2) (layer "F.Cu") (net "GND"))
 (segment (start 134.5725 79.3475) (end 121.3875 79.3475) (width 0.2) (layer "F.Cu") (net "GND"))
 (segment (start 176.4 93.635) (end 174.435 91.67) (width 0.2) (layer "F.Cu") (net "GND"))
 (segment (start 121.3875 79.3475) (end 112.98 87.755) (width 0.2) (layer "F.Cu") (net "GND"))
 (segment (start 176.4 97.102214) (end 176.4 93.635) (width 0.2) (layer "F.Cu") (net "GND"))
 (segment (start 144.79 108.7) (end 144.79 108.858) (width 0.2) (layer "F.Cu") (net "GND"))
 (segment (start 168.548 100.768) (end 168.56 100.78) (width 0.2) (layer "F.Cu") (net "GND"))
 (segment (start 153.492 98.228) (end 153.38 98.34) (width 0.2) (layer "F.Cu") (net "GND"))
 (segment (start 171.528 97.812) (end 175.690214 97.812) (width 0.2) (layer "F.Cu") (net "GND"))
 (segment (start 166.882 100.768) (end 164.342 98.228) (width 0.2) (layer "F.Cu") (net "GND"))
 (segment (start 153.38 98.34) (end 153.38 103.07) (width 0.2) (layer "F.Cu") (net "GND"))
 (segment (start 148.51 119.14) (end 149.66 117.99) (width 0.2) (layer "F.Cu") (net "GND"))
 (segment (start 149.66 122.66) (end 132.213402 122.66) (width 0.2) (layer "F.Cu") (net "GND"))
 (segment (start 144.791 109.259) (end 144.79 109.258) (width 0.2) (layer "F.Cu") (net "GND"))
 (segment (start 152.2 120.12) (end 149.66 122.66) (width 0.2) (layer "F.Cu") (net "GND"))
 (segment (start 147.192 109.258) (end 144.79 109.258) (width 0.2) (layer "F.Cu") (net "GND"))
 (segment (start 149.66 117.99) (end 152.2 117.99) (width 0.2) (layer "F.Cu") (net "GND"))
 (segment (start 152.2 117.99) (end 152.2 120.12) (width 0.2) (layer "F.Cu") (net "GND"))
 (segment (start 117.763402 108.21) (end 113.17 108.21) (width 0.2) (layer "F.Cu") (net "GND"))
 (segment (start 175.690214 97.812) (end 176.4 97.102214) (width 0.2) (layer "F.Cu") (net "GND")))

